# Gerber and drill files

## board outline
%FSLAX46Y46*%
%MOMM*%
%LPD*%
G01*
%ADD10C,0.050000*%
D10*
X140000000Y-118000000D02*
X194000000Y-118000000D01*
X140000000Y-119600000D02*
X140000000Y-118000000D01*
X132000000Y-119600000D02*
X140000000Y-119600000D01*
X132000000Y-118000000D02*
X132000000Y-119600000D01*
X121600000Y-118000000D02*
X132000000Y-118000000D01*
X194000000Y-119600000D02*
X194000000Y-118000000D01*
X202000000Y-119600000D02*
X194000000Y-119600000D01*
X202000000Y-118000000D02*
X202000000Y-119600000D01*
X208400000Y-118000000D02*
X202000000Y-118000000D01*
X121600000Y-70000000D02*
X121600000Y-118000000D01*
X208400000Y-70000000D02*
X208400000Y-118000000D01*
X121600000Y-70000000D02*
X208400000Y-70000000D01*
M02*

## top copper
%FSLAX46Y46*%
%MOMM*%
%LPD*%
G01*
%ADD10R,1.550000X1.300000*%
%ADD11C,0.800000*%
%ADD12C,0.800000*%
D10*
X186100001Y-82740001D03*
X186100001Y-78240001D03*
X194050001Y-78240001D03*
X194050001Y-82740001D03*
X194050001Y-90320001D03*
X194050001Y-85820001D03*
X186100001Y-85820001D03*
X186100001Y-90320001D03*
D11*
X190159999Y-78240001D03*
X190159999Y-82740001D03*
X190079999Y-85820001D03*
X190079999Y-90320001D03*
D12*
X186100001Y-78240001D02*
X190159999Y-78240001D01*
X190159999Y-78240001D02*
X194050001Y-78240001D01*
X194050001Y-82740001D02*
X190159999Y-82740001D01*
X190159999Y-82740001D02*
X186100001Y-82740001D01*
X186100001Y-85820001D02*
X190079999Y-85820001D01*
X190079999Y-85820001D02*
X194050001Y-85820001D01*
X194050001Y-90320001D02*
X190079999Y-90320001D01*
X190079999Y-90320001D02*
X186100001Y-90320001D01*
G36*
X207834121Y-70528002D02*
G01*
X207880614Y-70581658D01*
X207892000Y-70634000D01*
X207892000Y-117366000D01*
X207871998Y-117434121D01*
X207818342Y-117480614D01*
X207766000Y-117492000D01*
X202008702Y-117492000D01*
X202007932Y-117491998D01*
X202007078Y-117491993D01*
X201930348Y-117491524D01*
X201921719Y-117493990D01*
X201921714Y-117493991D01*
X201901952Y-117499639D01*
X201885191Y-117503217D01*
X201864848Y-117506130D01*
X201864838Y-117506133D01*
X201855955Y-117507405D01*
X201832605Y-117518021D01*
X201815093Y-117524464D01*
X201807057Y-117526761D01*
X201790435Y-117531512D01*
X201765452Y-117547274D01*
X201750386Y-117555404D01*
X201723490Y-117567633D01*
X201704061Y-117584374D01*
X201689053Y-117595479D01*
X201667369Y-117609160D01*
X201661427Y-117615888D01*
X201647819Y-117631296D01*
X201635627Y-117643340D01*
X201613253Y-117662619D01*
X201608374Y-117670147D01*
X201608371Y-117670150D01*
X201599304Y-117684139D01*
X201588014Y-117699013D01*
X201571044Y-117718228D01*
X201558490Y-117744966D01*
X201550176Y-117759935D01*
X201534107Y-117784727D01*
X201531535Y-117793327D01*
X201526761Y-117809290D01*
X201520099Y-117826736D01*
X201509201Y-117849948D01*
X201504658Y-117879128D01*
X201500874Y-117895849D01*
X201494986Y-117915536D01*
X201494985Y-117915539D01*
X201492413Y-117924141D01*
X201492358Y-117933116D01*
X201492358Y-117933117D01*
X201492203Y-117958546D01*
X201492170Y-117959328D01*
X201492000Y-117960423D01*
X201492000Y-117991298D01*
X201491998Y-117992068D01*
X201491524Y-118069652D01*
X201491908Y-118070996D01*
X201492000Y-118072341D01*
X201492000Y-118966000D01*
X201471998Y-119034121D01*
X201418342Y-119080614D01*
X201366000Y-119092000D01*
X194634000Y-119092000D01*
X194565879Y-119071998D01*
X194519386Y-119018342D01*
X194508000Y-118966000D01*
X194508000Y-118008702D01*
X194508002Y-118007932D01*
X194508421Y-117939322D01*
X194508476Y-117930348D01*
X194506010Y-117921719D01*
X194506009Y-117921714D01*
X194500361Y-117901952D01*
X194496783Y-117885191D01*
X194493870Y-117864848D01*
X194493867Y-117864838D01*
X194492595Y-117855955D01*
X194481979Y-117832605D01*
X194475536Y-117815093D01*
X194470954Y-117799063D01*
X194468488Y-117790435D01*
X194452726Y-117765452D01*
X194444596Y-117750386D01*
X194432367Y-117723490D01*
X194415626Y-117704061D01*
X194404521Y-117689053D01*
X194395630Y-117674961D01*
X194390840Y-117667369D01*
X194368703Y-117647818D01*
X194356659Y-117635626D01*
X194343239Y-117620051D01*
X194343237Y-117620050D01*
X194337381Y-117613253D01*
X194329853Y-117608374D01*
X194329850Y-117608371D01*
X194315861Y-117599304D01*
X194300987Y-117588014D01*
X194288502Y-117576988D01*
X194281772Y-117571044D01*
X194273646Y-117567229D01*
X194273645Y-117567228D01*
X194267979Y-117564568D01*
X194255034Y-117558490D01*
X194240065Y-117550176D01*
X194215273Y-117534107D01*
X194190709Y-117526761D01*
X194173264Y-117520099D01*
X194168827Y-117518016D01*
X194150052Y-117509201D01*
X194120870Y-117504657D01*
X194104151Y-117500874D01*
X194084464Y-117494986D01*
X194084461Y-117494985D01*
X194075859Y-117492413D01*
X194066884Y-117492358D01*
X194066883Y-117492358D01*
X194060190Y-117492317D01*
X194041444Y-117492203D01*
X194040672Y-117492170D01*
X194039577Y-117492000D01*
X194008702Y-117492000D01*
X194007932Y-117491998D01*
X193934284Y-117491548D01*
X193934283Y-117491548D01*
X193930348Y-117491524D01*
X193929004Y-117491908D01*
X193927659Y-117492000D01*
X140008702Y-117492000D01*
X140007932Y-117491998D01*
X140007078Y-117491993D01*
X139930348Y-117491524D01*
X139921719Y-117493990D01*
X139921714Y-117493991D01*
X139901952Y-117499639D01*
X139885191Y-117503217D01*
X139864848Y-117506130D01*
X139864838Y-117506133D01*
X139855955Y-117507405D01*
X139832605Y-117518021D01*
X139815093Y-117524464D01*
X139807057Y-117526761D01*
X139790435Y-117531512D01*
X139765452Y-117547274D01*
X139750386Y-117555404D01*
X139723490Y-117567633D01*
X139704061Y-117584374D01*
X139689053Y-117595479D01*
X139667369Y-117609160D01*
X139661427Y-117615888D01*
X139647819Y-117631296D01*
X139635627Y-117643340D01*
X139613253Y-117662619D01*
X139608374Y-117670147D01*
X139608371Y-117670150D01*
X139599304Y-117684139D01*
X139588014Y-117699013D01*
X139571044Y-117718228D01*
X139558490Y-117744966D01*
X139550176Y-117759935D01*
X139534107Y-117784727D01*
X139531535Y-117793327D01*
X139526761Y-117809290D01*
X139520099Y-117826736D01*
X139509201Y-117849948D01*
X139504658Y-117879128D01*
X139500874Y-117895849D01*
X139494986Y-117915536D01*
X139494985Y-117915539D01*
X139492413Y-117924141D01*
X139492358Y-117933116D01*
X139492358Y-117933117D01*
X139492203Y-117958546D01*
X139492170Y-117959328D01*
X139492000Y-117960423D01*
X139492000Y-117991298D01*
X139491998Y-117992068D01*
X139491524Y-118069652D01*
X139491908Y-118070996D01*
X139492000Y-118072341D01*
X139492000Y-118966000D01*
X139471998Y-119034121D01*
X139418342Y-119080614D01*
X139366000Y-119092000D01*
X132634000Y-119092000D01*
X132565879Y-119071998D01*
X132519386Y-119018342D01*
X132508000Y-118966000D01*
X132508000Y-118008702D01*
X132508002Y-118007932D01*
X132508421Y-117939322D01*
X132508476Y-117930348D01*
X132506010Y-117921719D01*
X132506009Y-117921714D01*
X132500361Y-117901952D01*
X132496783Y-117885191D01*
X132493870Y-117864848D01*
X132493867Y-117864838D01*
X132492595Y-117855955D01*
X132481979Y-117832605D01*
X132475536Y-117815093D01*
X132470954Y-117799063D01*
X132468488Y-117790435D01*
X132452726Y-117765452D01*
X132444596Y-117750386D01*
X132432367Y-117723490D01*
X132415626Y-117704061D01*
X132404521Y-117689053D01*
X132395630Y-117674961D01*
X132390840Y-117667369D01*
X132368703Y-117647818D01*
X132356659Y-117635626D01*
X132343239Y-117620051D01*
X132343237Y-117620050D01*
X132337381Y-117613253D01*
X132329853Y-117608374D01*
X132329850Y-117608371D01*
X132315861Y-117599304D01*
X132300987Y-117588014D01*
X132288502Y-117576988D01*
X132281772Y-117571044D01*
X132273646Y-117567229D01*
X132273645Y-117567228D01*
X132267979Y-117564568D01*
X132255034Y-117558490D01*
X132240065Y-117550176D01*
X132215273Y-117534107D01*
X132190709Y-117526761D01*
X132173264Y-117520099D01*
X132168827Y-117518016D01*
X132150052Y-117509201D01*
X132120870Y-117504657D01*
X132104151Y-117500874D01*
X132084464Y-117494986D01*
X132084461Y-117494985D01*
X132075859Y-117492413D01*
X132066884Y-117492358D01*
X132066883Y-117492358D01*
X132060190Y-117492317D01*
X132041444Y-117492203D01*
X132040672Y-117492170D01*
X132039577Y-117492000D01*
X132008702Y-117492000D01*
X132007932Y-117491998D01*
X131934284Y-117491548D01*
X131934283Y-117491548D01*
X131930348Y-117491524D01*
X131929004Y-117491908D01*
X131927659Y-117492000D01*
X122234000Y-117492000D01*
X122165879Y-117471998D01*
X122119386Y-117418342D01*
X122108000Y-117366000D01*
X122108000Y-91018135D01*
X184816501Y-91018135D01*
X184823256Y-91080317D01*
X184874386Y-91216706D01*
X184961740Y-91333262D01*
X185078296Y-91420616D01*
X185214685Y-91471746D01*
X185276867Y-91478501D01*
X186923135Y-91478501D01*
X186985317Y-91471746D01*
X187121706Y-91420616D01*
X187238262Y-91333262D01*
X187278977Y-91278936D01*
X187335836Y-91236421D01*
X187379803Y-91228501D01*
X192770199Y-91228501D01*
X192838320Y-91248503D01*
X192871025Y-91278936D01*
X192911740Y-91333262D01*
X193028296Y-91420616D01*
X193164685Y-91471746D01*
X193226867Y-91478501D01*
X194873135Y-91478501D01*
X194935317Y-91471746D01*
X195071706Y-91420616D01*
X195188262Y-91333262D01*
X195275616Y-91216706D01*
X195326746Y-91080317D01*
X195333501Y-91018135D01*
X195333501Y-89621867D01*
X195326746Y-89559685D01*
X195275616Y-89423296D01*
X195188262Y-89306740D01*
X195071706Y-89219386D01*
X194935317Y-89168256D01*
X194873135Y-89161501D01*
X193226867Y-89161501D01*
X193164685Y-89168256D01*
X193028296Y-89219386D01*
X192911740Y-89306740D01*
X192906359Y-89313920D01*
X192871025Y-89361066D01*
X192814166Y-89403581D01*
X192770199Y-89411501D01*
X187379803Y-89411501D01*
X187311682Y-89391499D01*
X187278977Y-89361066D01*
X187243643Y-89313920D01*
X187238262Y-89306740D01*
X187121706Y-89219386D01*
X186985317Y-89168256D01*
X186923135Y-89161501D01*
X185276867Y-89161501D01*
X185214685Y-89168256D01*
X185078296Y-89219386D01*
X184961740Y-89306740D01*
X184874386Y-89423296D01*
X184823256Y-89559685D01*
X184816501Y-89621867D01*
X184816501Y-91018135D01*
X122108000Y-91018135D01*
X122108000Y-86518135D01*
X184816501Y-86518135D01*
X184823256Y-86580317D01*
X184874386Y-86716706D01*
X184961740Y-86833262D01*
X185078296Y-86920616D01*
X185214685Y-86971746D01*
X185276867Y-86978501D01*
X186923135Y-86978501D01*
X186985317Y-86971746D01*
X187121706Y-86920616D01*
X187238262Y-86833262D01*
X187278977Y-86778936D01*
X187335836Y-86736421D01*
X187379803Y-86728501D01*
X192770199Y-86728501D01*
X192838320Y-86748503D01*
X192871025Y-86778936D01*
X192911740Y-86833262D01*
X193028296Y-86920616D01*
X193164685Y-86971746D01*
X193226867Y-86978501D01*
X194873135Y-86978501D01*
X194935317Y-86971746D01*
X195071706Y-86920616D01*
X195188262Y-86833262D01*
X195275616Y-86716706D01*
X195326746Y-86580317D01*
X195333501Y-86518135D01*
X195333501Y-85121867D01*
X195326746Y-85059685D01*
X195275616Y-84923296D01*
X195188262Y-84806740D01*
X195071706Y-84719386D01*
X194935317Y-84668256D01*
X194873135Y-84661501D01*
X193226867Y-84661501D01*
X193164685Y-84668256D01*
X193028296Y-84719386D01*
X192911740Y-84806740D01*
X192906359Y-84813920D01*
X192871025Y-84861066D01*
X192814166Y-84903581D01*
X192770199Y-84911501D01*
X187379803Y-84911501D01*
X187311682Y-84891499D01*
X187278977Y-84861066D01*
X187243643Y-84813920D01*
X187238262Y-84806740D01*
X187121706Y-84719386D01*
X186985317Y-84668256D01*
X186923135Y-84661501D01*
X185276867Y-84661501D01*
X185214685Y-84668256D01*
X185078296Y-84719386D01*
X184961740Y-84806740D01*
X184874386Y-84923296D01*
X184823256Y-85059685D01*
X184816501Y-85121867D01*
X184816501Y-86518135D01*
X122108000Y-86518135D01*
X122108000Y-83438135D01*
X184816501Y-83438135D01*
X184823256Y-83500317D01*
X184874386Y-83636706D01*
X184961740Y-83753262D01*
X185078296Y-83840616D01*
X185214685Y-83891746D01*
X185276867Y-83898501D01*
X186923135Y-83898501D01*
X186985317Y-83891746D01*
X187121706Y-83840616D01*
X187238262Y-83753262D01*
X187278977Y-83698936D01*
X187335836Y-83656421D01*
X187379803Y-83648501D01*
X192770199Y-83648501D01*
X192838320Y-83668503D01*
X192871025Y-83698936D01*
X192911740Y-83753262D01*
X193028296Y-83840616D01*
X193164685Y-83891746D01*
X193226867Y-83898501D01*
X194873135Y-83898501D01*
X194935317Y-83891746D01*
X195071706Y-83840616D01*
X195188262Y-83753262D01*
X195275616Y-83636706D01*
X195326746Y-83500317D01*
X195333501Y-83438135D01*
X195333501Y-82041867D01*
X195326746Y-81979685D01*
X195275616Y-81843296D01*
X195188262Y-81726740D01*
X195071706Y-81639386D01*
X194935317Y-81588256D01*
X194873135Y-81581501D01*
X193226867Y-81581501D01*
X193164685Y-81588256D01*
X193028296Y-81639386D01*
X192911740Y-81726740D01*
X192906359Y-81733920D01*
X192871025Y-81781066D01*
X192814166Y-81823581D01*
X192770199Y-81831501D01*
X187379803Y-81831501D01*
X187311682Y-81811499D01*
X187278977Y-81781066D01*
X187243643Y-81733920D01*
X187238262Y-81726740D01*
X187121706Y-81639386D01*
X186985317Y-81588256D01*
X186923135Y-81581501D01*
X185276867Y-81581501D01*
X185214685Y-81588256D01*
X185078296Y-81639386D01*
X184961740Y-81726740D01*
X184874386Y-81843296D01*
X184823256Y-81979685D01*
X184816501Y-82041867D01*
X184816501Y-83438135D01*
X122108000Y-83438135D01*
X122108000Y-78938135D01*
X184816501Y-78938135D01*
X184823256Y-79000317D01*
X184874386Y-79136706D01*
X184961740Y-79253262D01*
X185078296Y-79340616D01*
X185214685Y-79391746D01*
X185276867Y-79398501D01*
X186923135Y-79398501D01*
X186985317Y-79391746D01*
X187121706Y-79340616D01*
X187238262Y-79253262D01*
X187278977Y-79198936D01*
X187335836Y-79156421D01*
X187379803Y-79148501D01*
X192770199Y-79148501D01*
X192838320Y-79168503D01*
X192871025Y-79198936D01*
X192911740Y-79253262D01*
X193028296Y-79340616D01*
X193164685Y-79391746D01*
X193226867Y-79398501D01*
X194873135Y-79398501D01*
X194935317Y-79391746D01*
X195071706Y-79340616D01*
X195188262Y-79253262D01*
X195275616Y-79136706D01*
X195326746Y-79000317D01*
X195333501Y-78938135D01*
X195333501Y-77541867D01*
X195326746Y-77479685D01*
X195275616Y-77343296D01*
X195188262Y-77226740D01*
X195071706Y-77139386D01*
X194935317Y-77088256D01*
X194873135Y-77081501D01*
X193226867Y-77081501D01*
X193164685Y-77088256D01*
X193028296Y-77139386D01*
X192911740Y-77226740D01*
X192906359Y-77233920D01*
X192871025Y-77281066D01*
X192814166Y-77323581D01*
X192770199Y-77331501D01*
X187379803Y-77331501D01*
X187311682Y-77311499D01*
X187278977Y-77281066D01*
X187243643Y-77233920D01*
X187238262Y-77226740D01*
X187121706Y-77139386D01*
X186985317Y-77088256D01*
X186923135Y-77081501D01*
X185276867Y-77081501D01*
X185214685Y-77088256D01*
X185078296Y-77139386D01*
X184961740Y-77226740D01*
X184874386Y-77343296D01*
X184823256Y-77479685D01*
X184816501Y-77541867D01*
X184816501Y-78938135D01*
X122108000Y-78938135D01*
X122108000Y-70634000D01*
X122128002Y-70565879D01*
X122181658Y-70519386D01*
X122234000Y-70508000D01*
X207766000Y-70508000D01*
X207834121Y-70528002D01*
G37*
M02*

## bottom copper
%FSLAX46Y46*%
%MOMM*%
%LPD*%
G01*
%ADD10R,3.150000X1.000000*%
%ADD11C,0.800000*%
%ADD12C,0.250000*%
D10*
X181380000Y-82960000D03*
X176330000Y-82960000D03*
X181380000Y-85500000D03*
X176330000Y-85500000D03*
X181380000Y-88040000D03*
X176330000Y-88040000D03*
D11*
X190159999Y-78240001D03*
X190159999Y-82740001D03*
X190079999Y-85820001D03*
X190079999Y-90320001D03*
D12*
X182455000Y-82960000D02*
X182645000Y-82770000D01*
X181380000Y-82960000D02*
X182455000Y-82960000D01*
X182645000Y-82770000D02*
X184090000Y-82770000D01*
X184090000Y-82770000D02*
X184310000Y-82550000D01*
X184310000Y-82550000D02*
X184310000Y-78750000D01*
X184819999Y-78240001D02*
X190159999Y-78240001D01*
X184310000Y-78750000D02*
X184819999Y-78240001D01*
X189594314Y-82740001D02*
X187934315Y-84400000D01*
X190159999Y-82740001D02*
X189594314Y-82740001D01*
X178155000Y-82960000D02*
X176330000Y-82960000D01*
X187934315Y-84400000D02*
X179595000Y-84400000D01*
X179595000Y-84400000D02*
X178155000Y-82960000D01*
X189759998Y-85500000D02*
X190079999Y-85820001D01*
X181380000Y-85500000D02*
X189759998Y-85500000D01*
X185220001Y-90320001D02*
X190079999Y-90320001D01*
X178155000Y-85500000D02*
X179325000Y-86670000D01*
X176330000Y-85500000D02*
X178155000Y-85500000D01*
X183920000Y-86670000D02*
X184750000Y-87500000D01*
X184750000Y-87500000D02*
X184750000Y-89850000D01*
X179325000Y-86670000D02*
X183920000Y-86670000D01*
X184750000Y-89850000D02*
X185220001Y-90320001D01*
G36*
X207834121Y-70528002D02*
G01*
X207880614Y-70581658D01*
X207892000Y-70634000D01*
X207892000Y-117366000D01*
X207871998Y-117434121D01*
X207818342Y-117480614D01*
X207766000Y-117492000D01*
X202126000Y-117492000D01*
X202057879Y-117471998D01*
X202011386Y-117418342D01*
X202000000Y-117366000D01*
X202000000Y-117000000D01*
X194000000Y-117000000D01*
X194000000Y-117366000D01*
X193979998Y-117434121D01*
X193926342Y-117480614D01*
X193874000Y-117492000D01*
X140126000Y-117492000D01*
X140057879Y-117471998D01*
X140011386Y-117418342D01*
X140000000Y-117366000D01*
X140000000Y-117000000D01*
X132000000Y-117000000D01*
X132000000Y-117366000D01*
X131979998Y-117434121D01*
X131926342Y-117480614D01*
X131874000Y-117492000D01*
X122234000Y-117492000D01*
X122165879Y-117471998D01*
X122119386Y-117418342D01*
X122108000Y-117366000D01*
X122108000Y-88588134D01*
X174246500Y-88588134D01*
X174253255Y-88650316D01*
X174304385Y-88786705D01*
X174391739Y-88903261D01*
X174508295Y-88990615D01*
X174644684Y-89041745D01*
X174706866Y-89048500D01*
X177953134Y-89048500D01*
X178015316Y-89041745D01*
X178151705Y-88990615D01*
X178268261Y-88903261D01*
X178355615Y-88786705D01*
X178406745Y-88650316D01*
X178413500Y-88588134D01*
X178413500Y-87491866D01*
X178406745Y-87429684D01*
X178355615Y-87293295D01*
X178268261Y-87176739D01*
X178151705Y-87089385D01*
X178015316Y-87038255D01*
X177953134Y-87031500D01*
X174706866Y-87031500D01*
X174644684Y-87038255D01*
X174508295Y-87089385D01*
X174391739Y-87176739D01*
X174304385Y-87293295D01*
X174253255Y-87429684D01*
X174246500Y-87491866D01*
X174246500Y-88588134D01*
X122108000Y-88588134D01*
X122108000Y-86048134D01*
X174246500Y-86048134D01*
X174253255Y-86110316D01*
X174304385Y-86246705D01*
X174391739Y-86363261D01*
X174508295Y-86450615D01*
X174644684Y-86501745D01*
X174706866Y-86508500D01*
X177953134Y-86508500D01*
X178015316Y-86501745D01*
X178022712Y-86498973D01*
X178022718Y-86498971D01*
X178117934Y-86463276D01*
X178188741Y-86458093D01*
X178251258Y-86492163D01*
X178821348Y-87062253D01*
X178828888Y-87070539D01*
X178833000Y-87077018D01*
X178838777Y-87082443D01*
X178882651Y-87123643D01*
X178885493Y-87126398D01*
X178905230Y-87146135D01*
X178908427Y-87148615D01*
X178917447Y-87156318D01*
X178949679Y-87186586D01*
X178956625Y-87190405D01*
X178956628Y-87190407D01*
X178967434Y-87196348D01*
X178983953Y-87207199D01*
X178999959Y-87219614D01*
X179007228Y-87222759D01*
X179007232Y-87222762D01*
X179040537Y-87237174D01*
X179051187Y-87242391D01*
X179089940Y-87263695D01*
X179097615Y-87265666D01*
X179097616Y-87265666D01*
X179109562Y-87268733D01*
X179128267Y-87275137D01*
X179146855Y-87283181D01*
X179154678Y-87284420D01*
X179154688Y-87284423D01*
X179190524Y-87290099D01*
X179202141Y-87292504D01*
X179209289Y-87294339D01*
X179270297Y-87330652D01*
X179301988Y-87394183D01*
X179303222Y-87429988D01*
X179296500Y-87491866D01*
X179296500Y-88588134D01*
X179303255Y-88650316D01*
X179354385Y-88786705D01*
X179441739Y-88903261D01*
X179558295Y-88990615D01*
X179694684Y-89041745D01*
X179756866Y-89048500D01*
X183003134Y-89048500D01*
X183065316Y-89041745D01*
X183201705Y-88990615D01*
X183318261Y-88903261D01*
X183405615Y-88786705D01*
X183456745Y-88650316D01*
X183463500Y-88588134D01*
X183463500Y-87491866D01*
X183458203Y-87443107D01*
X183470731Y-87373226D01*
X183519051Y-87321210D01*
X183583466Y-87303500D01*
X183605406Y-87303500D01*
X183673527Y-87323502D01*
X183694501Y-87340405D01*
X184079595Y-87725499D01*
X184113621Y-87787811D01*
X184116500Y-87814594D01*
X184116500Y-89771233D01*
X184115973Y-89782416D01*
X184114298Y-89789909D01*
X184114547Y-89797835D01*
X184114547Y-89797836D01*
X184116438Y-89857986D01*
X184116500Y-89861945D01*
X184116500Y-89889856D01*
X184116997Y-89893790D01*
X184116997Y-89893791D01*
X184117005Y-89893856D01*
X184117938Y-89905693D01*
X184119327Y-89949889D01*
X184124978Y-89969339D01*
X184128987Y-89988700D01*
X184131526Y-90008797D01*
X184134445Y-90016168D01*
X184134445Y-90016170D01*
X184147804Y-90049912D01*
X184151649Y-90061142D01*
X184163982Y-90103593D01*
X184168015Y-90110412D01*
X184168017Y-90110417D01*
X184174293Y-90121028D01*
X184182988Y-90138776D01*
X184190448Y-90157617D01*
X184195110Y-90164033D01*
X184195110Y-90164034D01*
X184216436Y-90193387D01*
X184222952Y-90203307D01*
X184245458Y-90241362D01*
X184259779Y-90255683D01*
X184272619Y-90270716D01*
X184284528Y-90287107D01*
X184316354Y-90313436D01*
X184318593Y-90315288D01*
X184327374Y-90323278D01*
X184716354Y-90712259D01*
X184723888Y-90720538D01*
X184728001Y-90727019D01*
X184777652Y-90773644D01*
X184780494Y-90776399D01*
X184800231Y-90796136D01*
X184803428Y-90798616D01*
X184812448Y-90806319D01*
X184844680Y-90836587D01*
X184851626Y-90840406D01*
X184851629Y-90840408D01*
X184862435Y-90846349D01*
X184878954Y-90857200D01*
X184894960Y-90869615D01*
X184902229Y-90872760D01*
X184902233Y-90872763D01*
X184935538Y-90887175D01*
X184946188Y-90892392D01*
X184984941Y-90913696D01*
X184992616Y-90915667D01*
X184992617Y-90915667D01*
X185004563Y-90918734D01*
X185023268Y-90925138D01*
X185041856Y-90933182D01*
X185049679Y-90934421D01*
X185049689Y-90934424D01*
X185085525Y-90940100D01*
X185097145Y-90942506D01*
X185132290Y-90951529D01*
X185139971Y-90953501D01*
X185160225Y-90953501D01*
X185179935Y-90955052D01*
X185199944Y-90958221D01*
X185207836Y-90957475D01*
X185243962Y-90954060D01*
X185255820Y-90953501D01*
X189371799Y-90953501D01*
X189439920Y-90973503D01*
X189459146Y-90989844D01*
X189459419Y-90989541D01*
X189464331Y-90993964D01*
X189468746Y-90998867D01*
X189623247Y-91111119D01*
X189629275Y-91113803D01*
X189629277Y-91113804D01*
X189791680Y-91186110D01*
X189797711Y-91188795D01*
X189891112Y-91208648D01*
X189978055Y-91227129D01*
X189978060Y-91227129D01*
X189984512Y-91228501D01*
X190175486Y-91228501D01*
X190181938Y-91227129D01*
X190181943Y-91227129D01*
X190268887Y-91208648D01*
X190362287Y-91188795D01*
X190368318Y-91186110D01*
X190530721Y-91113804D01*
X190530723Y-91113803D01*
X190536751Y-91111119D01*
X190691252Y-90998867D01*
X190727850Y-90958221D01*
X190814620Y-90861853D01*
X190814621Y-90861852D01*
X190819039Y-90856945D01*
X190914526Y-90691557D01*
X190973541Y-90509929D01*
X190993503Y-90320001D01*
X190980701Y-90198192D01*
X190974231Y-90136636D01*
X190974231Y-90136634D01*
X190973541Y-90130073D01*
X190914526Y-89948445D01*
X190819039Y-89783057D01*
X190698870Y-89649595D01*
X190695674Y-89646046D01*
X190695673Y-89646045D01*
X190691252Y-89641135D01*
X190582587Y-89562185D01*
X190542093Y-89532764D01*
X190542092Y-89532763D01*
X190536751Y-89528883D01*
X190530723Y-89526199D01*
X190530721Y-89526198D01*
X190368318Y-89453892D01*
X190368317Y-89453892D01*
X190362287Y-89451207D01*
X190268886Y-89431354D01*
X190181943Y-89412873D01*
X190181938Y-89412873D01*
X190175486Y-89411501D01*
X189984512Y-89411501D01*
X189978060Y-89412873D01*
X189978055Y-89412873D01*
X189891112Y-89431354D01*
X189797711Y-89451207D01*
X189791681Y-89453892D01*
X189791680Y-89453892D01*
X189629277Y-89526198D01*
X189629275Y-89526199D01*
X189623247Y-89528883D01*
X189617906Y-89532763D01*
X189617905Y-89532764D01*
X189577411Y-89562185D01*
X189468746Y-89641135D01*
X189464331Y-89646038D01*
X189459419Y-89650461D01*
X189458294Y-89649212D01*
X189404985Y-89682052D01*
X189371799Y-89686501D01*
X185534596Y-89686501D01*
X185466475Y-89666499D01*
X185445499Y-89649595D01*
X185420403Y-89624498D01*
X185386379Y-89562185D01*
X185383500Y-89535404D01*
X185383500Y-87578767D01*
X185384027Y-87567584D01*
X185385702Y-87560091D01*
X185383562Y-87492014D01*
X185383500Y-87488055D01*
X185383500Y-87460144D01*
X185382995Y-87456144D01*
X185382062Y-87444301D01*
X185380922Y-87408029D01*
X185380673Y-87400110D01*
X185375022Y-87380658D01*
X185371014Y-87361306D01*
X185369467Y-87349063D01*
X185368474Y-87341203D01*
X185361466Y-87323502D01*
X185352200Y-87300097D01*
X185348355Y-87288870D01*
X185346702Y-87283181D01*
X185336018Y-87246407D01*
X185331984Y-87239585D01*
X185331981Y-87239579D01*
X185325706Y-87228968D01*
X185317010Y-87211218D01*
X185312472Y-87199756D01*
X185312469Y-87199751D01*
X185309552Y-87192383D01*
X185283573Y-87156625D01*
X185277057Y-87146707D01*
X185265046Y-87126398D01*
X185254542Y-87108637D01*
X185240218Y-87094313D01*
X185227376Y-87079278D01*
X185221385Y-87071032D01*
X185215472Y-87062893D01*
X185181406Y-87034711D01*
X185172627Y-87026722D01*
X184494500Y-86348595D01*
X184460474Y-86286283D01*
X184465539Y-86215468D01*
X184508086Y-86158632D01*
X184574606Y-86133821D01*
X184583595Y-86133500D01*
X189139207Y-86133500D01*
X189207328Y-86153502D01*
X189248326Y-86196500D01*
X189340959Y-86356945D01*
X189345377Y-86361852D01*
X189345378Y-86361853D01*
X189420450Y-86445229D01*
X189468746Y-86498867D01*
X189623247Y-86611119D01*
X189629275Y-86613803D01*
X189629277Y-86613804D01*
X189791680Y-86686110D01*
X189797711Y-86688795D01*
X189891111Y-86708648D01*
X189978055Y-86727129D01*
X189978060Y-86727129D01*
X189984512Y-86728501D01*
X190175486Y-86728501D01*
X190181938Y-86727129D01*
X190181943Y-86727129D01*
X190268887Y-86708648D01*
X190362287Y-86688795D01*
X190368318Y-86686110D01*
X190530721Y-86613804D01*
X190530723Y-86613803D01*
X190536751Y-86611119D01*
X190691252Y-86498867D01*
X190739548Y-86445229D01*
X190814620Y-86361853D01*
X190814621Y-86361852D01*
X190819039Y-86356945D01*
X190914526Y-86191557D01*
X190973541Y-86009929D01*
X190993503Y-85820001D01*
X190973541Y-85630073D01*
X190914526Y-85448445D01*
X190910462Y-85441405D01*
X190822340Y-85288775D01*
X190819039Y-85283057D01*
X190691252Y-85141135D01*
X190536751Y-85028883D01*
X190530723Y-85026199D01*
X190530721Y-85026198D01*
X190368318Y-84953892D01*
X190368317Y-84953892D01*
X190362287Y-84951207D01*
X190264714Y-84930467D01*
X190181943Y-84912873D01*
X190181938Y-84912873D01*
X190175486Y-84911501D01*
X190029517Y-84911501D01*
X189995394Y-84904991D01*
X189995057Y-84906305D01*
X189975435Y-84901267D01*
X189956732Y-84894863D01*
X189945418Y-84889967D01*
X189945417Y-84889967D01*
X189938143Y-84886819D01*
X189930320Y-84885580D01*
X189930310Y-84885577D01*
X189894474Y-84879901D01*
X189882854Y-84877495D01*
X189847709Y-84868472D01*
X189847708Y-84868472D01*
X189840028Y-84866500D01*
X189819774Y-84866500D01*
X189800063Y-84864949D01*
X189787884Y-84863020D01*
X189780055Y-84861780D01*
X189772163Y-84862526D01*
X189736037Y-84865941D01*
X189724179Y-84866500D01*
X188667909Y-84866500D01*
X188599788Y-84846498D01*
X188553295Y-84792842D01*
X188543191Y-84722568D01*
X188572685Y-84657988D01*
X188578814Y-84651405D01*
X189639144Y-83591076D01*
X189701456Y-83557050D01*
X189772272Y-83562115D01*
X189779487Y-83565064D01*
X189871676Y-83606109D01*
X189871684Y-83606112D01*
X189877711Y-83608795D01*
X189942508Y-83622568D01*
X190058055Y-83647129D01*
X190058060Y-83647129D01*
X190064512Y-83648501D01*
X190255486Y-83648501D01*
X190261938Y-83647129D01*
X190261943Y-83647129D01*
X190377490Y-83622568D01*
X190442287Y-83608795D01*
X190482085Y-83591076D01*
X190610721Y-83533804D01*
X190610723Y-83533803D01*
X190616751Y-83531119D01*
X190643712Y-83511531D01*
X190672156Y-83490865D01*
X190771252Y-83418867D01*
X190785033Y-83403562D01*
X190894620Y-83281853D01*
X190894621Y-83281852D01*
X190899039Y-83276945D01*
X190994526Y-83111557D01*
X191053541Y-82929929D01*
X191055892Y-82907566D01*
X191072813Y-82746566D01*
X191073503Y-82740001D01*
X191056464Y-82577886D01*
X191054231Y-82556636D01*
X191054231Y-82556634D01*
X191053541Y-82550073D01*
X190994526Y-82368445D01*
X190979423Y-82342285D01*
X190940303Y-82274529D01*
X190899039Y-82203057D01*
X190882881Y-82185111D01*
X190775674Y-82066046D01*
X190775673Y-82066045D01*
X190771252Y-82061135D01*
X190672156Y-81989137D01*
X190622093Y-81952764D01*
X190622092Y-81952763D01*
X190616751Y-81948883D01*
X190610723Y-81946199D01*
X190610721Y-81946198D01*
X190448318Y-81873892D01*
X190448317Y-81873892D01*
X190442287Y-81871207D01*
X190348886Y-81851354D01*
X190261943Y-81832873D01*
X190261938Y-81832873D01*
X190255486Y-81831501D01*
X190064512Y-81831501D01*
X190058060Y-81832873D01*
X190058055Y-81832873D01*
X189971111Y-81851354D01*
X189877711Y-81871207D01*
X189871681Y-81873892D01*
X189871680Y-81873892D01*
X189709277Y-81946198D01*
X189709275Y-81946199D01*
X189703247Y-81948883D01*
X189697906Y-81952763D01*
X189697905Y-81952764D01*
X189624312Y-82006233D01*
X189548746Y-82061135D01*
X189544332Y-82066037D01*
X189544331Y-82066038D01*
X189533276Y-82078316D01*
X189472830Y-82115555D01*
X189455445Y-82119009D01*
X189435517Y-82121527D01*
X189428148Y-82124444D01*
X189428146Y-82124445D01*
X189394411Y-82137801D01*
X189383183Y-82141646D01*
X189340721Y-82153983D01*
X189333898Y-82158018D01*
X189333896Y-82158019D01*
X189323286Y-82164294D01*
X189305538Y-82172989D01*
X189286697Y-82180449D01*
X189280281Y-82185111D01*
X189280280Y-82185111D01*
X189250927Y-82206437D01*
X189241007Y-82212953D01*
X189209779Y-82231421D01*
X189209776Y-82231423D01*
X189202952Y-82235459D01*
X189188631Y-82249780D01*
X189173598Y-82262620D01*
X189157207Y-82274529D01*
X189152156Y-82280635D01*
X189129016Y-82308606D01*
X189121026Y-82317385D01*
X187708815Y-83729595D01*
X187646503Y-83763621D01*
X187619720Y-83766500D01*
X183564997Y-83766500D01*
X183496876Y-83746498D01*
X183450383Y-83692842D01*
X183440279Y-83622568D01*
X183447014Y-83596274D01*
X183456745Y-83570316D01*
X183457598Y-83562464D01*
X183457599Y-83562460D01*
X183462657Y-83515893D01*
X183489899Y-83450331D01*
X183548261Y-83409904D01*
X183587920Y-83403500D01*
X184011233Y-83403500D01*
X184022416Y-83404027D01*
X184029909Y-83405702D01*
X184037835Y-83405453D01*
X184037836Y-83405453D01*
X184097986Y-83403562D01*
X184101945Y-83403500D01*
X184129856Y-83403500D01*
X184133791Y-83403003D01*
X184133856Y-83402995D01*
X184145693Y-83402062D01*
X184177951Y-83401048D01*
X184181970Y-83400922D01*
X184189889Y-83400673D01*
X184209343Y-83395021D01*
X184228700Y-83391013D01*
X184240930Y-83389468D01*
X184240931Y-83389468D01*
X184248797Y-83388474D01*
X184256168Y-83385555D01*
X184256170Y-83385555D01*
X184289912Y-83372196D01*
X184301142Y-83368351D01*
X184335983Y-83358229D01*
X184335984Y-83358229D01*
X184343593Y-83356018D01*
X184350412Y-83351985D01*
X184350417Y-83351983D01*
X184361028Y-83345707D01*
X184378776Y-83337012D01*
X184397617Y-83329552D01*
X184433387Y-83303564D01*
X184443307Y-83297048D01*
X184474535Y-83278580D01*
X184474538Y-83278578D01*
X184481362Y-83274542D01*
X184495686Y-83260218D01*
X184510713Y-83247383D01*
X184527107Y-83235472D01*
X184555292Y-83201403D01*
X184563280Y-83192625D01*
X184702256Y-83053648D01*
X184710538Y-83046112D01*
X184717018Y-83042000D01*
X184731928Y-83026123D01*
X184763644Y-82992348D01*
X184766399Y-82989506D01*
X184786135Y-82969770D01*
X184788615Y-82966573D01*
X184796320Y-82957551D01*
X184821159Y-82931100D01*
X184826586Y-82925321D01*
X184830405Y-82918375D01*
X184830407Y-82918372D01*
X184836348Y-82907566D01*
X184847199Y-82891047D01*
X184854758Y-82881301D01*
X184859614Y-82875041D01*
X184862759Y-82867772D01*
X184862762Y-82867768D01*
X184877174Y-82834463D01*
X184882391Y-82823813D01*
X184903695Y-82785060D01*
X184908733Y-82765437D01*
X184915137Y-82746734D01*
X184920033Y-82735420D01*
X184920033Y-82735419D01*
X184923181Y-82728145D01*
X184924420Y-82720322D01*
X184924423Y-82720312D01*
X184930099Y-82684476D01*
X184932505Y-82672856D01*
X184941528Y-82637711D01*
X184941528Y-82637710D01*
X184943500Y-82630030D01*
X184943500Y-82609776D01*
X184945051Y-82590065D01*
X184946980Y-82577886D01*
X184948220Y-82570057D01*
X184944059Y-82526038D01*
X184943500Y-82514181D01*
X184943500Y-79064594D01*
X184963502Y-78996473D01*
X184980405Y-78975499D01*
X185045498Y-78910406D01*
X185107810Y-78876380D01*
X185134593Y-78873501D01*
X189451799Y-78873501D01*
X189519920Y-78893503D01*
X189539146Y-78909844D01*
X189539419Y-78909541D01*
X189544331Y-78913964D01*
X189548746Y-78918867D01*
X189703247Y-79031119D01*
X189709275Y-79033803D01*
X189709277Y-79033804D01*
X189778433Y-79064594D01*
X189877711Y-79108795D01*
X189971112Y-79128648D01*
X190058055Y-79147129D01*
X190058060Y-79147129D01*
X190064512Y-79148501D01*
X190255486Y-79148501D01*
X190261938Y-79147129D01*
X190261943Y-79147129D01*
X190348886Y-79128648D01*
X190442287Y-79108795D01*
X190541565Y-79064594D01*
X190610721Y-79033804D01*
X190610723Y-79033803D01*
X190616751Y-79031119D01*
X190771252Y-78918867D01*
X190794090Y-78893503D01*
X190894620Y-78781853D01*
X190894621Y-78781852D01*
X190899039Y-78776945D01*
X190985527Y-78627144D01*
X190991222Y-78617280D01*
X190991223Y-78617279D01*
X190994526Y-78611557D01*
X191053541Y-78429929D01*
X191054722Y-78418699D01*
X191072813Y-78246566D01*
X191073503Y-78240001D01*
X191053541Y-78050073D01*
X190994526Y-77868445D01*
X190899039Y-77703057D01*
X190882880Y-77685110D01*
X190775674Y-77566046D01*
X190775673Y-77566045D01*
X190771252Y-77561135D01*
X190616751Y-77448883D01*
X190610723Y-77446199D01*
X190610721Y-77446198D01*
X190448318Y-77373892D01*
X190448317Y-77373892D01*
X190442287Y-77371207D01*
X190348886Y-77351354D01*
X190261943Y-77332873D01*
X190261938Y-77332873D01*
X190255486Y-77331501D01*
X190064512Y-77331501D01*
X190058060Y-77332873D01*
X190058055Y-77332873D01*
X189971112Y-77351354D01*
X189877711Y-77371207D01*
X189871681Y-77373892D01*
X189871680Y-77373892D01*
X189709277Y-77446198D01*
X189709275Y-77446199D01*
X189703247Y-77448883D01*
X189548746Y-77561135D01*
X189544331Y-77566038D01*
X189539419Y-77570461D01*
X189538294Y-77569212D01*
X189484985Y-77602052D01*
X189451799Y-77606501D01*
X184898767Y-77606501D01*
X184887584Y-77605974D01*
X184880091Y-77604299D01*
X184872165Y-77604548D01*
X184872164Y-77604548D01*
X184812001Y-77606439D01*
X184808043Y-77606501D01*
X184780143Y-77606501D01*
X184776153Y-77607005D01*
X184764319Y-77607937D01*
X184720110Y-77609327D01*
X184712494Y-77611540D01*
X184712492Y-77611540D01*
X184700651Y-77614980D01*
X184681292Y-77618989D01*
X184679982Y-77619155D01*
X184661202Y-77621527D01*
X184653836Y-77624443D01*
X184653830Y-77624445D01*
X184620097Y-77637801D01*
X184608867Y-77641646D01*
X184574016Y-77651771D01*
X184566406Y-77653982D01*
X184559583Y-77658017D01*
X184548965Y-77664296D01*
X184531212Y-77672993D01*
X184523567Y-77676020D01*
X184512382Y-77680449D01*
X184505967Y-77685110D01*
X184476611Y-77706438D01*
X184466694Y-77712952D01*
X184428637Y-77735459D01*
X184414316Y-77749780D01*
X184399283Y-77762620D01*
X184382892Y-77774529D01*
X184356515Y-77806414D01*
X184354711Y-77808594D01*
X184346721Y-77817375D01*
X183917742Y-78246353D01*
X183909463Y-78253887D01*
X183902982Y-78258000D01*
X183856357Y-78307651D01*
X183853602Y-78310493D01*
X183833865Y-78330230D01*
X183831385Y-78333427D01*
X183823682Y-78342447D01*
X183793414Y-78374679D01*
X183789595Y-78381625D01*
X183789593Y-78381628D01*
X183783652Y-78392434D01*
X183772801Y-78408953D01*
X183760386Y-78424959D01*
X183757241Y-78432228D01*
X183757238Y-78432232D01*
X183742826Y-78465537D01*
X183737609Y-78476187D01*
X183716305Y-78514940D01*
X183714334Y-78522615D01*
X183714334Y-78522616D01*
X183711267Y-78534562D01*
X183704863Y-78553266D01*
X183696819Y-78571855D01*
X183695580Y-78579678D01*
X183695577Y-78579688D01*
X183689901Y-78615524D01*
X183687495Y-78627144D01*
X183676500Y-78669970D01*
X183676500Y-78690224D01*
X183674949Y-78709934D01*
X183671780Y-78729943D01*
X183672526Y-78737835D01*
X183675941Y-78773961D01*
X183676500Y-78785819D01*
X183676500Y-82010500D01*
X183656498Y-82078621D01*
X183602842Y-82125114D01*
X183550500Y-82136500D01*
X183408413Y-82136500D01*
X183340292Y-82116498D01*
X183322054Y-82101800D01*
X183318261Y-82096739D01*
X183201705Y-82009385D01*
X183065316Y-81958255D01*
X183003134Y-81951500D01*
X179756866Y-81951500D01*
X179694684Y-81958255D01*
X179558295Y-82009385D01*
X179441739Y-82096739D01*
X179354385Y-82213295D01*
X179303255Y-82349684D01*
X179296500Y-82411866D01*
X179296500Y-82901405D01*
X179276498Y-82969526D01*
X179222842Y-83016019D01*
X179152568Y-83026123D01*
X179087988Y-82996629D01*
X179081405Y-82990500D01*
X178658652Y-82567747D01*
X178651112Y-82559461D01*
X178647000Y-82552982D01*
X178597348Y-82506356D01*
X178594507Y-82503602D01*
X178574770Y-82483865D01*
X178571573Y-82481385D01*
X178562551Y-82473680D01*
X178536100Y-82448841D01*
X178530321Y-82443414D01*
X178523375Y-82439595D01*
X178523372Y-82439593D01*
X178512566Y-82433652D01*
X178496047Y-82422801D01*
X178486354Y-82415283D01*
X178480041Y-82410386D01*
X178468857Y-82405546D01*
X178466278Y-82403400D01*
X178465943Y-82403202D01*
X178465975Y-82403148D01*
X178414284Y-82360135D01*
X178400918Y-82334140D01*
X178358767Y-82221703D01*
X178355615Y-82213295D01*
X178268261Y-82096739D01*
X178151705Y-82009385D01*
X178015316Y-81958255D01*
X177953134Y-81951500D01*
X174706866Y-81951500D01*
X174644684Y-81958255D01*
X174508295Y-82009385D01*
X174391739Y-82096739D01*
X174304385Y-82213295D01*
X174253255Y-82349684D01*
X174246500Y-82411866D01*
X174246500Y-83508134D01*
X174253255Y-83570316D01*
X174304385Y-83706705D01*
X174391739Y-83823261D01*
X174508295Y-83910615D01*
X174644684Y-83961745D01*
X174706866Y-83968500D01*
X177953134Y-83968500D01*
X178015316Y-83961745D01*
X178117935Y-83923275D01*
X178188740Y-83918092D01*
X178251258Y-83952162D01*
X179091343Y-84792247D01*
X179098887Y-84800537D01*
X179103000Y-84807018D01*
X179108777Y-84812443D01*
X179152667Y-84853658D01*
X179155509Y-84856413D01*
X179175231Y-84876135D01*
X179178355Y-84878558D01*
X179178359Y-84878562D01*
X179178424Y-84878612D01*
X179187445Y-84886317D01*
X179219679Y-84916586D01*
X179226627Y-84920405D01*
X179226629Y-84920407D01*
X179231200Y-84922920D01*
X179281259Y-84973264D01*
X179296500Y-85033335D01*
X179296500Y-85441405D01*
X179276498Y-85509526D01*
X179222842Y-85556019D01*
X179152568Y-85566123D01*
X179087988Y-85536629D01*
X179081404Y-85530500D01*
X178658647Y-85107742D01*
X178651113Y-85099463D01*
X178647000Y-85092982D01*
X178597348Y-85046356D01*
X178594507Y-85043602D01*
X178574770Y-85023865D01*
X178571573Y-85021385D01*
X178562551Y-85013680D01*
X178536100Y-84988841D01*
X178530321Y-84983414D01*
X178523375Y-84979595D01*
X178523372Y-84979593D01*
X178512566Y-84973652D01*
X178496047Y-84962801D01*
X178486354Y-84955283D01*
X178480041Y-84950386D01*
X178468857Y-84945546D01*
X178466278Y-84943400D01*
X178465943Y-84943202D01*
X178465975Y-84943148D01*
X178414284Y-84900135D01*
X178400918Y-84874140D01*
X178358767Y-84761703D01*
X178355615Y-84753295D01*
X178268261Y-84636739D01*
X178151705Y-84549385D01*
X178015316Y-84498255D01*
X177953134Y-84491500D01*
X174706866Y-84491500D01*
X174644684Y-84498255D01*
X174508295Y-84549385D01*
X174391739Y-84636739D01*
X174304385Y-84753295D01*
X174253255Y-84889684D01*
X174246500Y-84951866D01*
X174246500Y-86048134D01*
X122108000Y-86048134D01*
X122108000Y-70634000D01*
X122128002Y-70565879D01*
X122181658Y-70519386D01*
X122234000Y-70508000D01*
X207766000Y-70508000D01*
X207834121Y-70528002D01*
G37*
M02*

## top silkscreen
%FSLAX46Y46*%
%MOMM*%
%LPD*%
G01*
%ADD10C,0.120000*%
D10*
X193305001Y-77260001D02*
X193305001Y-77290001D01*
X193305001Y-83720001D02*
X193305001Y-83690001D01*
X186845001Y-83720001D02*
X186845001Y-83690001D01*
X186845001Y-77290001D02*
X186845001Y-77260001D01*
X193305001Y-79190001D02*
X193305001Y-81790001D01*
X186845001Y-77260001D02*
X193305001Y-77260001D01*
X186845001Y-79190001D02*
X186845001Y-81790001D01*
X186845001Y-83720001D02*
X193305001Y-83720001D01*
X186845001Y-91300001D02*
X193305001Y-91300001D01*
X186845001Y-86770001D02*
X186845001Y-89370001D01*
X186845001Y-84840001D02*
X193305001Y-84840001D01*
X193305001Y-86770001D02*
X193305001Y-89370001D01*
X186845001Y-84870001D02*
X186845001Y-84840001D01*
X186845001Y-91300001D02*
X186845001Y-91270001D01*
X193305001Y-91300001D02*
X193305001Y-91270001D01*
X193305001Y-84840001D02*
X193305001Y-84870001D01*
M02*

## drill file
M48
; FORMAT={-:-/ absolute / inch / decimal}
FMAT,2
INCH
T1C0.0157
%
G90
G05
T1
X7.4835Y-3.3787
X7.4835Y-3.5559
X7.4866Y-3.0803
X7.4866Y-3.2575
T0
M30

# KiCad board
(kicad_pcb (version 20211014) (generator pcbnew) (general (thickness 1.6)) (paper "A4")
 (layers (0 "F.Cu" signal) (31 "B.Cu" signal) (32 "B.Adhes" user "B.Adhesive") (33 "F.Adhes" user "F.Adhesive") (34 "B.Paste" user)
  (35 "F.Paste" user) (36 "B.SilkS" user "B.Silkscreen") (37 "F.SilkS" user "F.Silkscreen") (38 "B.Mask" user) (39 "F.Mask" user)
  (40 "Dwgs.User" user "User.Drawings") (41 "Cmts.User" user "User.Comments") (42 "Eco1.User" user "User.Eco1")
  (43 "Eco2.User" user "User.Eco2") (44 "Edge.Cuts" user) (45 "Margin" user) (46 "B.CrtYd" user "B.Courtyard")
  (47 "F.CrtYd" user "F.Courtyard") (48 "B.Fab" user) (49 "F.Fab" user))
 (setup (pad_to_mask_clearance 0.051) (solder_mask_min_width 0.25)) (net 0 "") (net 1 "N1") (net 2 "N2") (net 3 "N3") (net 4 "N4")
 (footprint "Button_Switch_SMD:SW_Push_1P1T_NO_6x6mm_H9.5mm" (layer "F.Cu") (at 190.075001 80.490001)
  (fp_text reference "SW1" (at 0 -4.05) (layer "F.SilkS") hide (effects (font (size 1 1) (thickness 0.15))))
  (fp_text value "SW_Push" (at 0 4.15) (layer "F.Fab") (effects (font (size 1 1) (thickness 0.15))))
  (fp_line (start 3.23 -1.3) (end 3.23 1.3) (layer "F.SilkS") (width 0.12))
  (fp_line (start 3.23 3.23) (end 3.23 3.2) (layer "F.SilkS") (width 0.12))
  (fp_line (start -3.23 3.23) (end 3.23 3.23) (layer "F.SilkS") (width 0.12))
  (fp_line (start -3.23 -3.23) (end 3.23 -3.23) (layer "F.SilkS") (width 0.12))
  (fp_line (start 3.23 -3.23) (end 3.23 -3.2) (layer "F.SilkS") (width 0.12))
  (fp_line (start -3.23 3.23) (end -3.23 3.2) (layer "F.SilkS") (width 0.12))
  (fp_line (start -3.23 -1.3) (end -3.23 1.3) (layer "F.SilkS") (width 0.12))
  (fp_line (start -3.23 -3.2) (end -3.23 -3.23) (layer "F.SilkS") (width 0.12))
  (pad "1" smd rect locked (at -3.975 -2.25) (size 1.55 1.3) (layers "F.Cu" "F.Paste" "F.Mask") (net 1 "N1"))
  (pad "1" smd rect locked (at 3.975 -2.25) (size 1.55 1.3) (layers "F.Cu" "F.Paste" "F.Mask") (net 1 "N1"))
  (pad "2" smd rect locked (at -3.975 2.25) (size 1.55 1.3) (layers "F.Cu" "F.Paste" "F.Mask") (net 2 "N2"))
  (pad "2" smd rect locked (at 3.975 2.25) (size 1.55 1.3) (layers "F.Cu" "F.Paste" "F.Mask") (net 2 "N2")))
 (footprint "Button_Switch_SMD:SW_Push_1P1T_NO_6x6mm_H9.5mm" (layer "F.Cu") (at 190.075001 88.070001)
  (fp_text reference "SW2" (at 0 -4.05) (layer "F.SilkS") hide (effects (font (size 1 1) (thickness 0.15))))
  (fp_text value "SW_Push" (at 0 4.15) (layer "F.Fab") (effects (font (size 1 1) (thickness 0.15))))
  (fp_line (start -3.23 3.23) (end -3.23 3.2) (layer "F.SilkS") (width 0.12))
  (fp_line (start 3.23 -3.23) (end 3.23 -3.2) (layer "F.SilkS") (width 0.12))
  (fp_line (start -3.23 -1.3) (end -3.23 1.3) (layer "F.SilkS") (width 0.12))
  (fp_line (start -3.23 -3.2) (end -3.23 -3.23) (layer "F.SilkS") (width 0.12))
  (fp_line (start 3.23 -1.3) (end 3.23 1.3) (layer "F.SilkS") (width 0.12))
  (fp_line (start -3.23 3.23) (end 3.23 3.23) (layer "F.SilkS") (width 0.12))
  (fp_line (start 3.23 3.23) (end 3.23 3.2) (layer "F.SilkS") (width 0.12))
  (fp_line (start -3.23 -3.23) (end 3.23 -3.23) (layer "F.SilkS") (width 0.12))
  (pad "1" smd rect locked (at 3.975 -2.25) (size 1.55 1.3) (layers "F.Cu" "F.Paste" "F.Mask") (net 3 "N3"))
  (pad "1" smd rect locked (at -3.975 -2.25) (size 1.55 1.3) (layers "F.Cu" "F.Paste" "F.Mask") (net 3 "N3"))
  (pad "2" smd rect locked (at -3.975 2.25) (size 1.55 1.3) (layers "F.Cu" "F.Paste" "F.Mask") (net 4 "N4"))
  (pad "2" smd rect locked (at 3.975 2.25) (size 1.55 1.3) (layers "F.Cu" "F.Paste" "F.Mask") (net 4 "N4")))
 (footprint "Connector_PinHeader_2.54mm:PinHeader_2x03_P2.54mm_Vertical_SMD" (layer "B.Cu") (at 178.855 85.5 180)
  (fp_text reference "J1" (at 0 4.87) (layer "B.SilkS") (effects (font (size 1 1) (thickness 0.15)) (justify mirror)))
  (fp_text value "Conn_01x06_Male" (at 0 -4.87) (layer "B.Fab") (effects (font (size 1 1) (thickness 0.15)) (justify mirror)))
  (pad "1" smd rect locked (at -2.525 2.54 180) (size 3.15 1) (layers "B.Cu" "B.Paste" "B.Mask") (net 1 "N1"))
  (pad "2" smd rect locked (at 2.525 2.54 180) (size 3.15 1) (layers "B.Cu" "B.Paste" "B.Mask") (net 2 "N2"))
  (pad "3" smd rect locked (at -2.525 0 180) (size 3.15 1) (layers "B.Cu" "B.Paste" "B.Mask") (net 3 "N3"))
  (pad "4" smd rect locked (at 2.525 0 180) (size 3.15 1) (layers "B.Cu" "B.Paste" "B.Mask") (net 4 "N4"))
  (pad "5" smd rect locked (at -2.525 -2.54 180) (size 3.15 1) (layers "B.Cu" "B.Paste" "B.Mask"))
  (pad "6" smd rect locked (at 2.525 -2.54 180) (size 3.15 1) (layers "B.Cu" "B.Paste" "B.Mask")))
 (gr_line (start 140 118) (end 194 118) (layer "Edge.Cuts") (width 0.05))
 (gr_line (start 208.4 118) (end 202 118) (layer "Edge.Cuts") (width 0.05))
 (gr_line (start 208.4 70) (end 208.4 118) (layer "Edge.Cuts") (width 0.05))
 (gr_line (start 121.6 70) (end 121.6 118) (layer "Edge.Cuts") (width 0.05))
 (gr_line (start 132 119.6) (end 140 119.6) (layer "Edge.Cuts") (width 0.05))
 (gr_line (start 202 118) (end 202 119.6) (layer "Edge.Cuts") (width 0.05))
 (gr_line (start 132 118) (end 132 119.6) (layer "Edge.Cuts") (width 0.05))
 (gr_line (start 202 119.6) (end 194 119.6) (layer "Edge.Cuts") (width 0.05))
 (gr_line (start 194 119.6) (end 194 118) (layer "Edge.Cuts") (width 0.05))
 (gr_line (start 121.6 118) (end 132 118) (layer "Edge.Cuts") (width 0.05))
 (gr_line (start 140 119.6) (end 140 118) (layer "Edge.Cuts") (width 0.05))
 (gr_line (start 121.6 70) (end 208.4 70) (layer "Edge.Cuts") (width 0.05))
 (segment (start 190.159999 78.240001) (end 194.050001 78.240001) (width 0.8) (layer "F.Cu") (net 1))
 (segment (start 186.100001 78.240001) (end 190.159999 78.240001) (width 0.8) (layer "F.Cu") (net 1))
 (via (at 190.159999 78.240001) (size 0.8) (drill 0.4) (layers "F.Cu" "B.Cu") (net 1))
 (segment (start 182.645 82.77) (end 184.09 82.77) (width 0.25) (layer "B.Cu") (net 1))
 (segment (start 182.455 82.96) (end 182.645 82.77) (width 0.25) (layer "B.Cu") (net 1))
 (segment (start 184.31 82.55) (end 184.31 78.75) (width 0.25) (layer "B.Cu") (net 1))
 (segment (start 181.38 82.96) (end 182.455 82.96) (width 0.25) (layer "B.Cu") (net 1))
 (segment (start 184.09 82.77) (end 184.31 82.55) (width 0.25) (layer "B.Cu") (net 1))
 (segment (start 184.31 78.75) (end 184.819999 78.240001) (width 0.25) (layer "B.Cu") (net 1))
 (segment (start 184.819999 78.240001) (end 190.159999 78.240001) (width 0.25) (layer "B.Cu") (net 1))
 (segment (start 190.159999 82.740001) (end 186.100001 82.740001) (width 0.8) (layer "F.Cu") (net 2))
 (segment (start 194.050001 82.740001) (end 190.159999 82.740001) (width 0.8) (layer "F.Cu") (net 2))
 (via (at 190.159999 82.740001) (size 0.8) (drill 0.4) (layers "F.Cu" "B.Cu") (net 2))
 (segment (start 187.934315 84.4) (end 179.595 84.4) (width 0.25) (layer "B.Cu") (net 2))
 (segment (start 189.594314 82.740001) (end 187.934315 84.4) (width 0.25) (layer "B.Cu") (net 2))
 (segment (start 178.155 82.96) (end 176.33 82.96) (width 0.25) (layer "B.Cu") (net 2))
 (segment (start 190.159999 82.740001) (end 189.594314 82.740001) (width 0.25) (layer "B.Cu") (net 2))
 (segment (start 179.595 84.4) (end 178.155 82.96) (width 0.25) (layer "B.Cu") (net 2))
 (segment (start 190.079999 85.820001) (end 194.050001 85.820001) (width 0.8) (layer "F.Cu") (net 3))
 (segment (start 186.100001 85.820001) (end 190.079999 85.820001) (width 0.8) (layer "F.Cu") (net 3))
 (via (at 190.079999 85.820001) (size 0.8) (drill 0.4) (layers "F.Cu" "B.Cu") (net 3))
 (segment (start 189.759998 85.5) (end 190.079999 85.820001) (width 0.25) (layer "B.Cu") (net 3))
 (segment (start 181.38 85.5) (end 189.759998 85.5) (width 0.25) (layer "B.Cu") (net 3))
 (segment (start 190.079999 90.320001) (end 186.100001 90.320001) (width 0.8) (layer "F.Cu") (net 4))
 (segment (start 194.050001 90.320001) (end 190.079999 90.320001) (width 0.8) (layer "F.Cu") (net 4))
 (via (at 190.079999 90.320001) (size 0.8) (drill 0.4) (layers "F.Cu" "B.Cu") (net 4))
 (segment (start 179.325 86.67) (end 183.92 86.67) (width 0.25) (layer "B.Cu") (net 4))
 (segment (start 185.220001 90.320001) (end 190.079999 90.320001) (width 0.25) (layer "B.Cu") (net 4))
 (segment (start 183.92 86.67) (end 184.75 87.5) (width 0.25) (layer "B.Cu") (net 4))
 (segment (start 178.155 85.5) (end 179.325 86.67) (width 0.25) (layer "B.Cu") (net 4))
 (segment (start 176.33 85.5) (end 178.155 85.5) (width 0.25) (layer "B.Cu") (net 4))
 (segment (start 184.75 87.5) (end 184.75 89.85) (width 0.25) (layer "B.Cu") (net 4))
 (segment (start 184.75 89.85) (end 185.220001 90.320001) (width 0.25) (layer "B.Cu") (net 4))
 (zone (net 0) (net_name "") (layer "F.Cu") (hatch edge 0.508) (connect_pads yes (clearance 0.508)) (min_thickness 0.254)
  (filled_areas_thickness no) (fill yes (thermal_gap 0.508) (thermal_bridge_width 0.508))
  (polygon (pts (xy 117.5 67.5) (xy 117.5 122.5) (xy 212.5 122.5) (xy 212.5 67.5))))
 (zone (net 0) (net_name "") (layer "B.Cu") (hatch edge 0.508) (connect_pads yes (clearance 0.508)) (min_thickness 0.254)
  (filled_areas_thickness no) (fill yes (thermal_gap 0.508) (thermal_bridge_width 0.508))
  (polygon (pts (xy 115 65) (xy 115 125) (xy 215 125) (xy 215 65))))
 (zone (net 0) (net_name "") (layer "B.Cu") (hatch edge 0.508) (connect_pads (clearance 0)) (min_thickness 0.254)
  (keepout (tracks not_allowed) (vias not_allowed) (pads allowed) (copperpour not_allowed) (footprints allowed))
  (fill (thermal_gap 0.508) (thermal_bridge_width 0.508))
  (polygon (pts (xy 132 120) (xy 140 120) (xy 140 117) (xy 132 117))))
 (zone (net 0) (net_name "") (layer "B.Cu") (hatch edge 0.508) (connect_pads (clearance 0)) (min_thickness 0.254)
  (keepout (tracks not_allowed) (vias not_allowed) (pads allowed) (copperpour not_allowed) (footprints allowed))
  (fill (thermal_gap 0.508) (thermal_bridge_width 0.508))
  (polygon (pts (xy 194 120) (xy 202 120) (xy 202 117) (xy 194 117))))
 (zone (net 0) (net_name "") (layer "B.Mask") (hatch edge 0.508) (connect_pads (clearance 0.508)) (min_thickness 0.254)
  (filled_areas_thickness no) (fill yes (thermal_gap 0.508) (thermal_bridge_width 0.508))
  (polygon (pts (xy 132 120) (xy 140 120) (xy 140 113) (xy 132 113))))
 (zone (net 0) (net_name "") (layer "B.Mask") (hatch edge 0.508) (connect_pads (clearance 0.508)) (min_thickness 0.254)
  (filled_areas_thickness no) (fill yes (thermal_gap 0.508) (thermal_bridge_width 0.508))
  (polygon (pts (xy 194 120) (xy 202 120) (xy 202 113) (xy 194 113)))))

